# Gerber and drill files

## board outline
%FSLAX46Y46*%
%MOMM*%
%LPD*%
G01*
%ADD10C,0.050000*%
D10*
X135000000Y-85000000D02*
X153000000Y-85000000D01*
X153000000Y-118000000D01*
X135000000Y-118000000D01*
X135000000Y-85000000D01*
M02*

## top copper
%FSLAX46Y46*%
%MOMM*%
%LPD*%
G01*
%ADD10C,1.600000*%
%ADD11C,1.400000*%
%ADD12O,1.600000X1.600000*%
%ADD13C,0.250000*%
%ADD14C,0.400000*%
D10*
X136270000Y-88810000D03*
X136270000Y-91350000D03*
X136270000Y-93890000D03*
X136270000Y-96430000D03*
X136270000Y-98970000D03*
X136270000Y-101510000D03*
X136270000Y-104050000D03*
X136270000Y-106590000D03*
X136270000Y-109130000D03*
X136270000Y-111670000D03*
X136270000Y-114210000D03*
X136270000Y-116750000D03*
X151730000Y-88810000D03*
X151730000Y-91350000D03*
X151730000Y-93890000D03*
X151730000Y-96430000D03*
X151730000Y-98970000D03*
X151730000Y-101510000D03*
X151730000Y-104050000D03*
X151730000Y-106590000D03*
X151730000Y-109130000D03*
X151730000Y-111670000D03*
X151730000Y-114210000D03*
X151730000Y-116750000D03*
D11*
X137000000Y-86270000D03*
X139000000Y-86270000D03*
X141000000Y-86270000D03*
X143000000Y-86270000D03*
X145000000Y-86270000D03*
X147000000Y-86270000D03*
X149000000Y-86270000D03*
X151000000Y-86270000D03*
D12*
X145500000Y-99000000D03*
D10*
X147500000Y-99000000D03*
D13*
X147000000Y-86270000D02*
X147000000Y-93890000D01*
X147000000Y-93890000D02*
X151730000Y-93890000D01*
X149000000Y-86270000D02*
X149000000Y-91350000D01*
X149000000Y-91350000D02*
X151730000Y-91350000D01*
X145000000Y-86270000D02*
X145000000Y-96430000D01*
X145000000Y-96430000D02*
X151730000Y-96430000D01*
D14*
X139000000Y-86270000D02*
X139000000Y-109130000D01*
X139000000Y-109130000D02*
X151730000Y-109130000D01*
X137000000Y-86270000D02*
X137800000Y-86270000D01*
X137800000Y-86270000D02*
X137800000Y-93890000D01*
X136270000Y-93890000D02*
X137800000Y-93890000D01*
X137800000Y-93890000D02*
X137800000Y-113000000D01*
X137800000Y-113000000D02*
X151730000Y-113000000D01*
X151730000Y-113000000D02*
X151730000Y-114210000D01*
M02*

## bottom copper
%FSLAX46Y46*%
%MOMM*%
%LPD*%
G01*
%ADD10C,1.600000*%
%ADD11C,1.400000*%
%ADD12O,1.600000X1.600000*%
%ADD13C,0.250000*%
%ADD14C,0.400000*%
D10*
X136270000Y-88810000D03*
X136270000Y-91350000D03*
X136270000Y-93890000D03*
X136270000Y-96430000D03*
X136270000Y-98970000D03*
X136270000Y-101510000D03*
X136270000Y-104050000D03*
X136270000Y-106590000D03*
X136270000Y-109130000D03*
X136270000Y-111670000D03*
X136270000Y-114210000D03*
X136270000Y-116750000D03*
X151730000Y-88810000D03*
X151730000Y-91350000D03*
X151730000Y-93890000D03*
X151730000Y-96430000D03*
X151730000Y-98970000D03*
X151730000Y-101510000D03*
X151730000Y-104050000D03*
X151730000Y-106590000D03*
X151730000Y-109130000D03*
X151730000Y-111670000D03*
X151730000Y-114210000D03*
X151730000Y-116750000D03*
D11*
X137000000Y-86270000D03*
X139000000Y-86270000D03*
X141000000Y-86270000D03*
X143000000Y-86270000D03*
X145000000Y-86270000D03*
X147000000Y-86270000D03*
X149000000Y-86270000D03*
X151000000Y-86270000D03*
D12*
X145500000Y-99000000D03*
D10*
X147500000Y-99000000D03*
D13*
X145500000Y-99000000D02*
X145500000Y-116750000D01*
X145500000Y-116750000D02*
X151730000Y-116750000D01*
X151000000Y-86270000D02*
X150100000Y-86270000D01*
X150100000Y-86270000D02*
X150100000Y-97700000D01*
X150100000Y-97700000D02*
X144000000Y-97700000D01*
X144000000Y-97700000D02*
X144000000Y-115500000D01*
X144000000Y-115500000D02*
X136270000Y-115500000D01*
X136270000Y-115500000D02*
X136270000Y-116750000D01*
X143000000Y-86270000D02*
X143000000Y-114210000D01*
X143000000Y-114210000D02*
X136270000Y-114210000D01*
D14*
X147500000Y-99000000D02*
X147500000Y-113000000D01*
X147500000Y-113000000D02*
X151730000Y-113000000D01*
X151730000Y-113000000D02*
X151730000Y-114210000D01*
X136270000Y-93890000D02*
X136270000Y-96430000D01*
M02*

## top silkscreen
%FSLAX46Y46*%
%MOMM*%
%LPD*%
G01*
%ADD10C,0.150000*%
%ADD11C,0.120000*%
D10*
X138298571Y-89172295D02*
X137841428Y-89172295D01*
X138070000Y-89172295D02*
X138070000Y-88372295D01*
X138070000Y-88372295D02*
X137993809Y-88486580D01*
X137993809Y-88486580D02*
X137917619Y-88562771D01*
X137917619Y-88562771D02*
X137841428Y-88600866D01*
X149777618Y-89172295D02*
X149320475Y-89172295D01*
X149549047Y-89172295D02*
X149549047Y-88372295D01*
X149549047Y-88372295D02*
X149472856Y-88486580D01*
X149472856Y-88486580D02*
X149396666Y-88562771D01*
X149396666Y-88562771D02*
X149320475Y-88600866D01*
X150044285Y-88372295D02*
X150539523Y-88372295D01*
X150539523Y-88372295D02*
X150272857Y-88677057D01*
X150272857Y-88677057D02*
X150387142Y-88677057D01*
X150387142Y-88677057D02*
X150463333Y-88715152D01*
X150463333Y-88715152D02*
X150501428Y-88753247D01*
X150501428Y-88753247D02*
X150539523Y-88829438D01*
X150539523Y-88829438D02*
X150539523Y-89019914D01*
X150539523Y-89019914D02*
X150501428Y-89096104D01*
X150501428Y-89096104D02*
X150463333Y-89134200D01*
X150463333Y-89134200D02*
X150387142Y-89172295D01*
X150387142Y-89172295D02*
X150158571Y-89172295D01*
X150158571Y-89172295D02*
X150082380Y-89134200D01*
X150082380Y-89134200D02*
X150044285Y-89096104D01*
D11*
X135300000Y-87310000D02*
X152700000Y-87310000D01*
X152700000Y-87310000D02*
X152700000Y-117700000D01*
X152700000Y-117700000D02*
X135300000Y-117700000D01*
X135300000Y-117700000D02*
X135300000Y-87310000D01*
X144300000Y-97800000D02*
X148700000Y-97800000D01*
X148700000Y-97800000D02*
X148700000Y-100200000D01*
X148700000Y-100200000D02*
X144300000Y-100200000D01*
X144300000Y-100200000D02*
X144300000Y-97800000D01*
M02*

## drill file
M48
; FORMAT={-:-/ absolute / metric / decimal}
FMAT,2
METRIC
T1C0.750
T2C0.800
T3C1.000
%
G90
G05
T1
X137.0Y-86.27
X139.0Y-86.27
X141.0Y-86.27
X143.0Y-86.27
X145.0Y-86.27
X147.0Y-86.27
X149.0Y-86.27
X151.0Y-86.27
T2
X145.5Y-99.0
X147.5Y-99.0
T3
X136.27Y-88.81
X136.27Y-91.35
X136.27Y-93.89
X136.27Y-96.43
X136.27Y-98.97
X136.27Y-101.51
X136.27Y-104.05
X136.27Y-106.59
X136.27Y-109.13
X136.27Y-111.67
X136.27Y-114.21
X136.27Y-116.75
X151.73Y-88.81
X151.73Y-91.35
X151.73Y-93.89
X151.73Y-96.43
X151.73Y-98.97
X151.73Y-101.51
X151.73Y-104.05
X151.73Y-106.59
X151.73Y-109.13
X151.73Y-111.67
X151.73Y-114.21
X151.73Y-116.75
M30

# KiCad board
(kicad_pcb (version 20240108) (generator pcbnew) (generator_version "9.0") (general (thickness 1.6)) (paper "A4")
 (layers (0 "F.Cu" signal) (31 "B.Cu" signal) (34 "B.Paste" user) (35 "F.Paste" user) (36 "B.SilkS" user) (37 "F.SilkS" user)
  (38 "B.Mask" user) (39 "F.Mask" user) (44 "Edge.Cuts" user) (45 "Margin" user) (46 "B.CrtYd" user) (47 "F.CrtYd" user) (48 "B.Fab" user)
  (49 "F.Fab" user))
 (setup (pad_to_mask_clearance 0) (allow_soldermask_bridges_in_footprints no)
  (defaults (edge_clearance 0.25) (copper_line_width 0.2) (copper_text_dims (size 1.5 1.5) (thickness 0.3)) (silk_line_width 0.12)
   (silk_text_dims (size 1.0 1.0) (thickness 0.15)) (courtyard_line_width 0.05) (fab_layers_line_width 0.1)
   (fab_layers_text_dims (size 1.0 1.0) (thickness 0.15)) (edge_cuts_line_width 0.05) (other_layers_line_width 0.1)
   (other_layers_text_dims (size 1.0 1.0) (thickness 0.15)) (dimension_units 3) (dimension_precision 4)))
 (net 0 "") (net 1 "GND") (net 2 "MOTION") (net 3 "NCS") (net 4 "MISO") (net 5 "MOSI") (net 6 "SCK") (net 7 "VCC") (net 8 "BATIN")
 (gr_rect (start 135.0000 85.0000) (end 153.0000 118.0000) (stroke (width 0.05) (type default)) (layer "Edge.Cuts"))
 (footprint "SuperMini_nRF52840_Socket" (layer "F.Cu") (at 135.0000 85.0000)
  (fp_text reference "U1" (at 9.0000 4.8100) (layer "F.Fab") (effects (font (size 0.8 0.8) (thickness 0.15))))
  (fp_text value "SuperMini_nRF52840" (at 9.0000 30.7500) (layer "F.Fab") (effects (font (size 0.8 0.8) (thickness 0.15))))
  (pad "1" thru_hole circle (at 1.2700 3.8100) (size 1.6000 1.6000) (drill 1.0000) (layers "*.Cu" "*.Mask"))
  (pad "2" thru_hole circle (at 1.2700 6.3500) (size 1.6000 1.6000) (drill 1.0000) (layers "*.Cu" "*.Mask"))
  (pad "3" thru_hole circle (at 1.2700 8.8900) (size 1.6000 1.6000) (drill 1.0000) (layers "*.Cu" "*.Mask") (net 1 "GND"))
  (pad "4" thru_hole circle (at 1.2700 11.4300) (size 1.6000 1.6000) (drill 1.0000) (layers "*.Cu" "*.Mask") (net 1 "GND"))
  (pad "5" thru_hole circle (at 1.2700 13.9700) (size 1.6000 1.6000) (drill 1.0000) (layers "*.Cu" "*.Mask"))
  (pad "6" thru_hole circle (at 1.2700 16.5100) (size 1.6000 1.6000) (drill 1.0000) (layers "*.Cu" "*.Mask"))
  (pad "7" thru_hole circle (at 1.2700 19.0500) (size 1.6000 1.6000) (drill 1.0000) (layers "*.Cu" "*.Mask"))
  (pad "8" thru_hole circle (at 1.2700 21.5900) (size 1.6000 1.6000) (drill 1.0000) (layers "*.Cu" "*.Mask"))
  (pad "9" thru_hole circle (at 1.2700 24.1300) (size 1.6000 1.6000) (drill 1.0000) (layers "*.Cu" "*.Mask"))
  (pad "10" thru_hole circle (at 1.2700 26.6700) (size 1.6000 1.6000) (drill 1.0000) (layers "*.Cu" "*.Mask"))
  (pad "11" thru_hole circle (at 1.2700 29.2100) (size 1.6000 1.6000) (drill 1.0000) (layers "*.Cu" "*.Mask") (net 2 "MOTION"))
  (pad "12" thru_hole circle (at 1.2700 31.7500) (size 1.6000 1.6000) (drill 1.0000) (layers "*.Cu" "*.Mask") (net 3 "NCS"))
  (pad "13" thru_hole circle (at 16.7300 3.8100) (size 1.6000 1.6000) (drill 1.0000) (layers "*.Cu" "*.Mask"))
  (pad "14" thru_hole circle (at 16.7300 6.3500) (size 1.6000 1.6000) (drill 1.0000) (layers "*.Cu" "*.Mask") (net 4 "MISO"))
  (pad "15" thru_hole circle (at 16.7300 8.8900) (size 1.6000 1.6000) (drill 1.0000) (layers "*.Cu" "*.Mask") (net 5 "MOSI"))
  (pad "16" thru_hole circle (at 16.7300 11.4300) (size 1.6000 1.6000) (drill 1.0000) (layers "*.Cu" "*.Mask") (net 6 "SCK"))
  (pad "17" thru_hole circle (at 16.7300 13.9700) (size 1.6000 1.6000) (drill 1.0000) (layers "*.Cu" "*.Mask"))
  (pad "18" thru_hole circle (at 16.7300 16.5100) (size 1.6000 1.6000) (drill 1.0000) (layers "*.Cu" "*.Mask"))
  (pad "19" thru_hole circle (at 16.7300 19.0500) (size 1.6000 1.6000) (drill 1.0000) (layers "*.Cu" "*.Mask"))
  (pad "20" thru_hole circle (at 16.7300 21.5900) (size 1.6000 1.6000) (drill 1.0000) (layers "*.Cu" "*.Mask"))
  (pad "21" thru_hole circle (at 16.7300 24.1300) (size 1.6000 1.6000) (drill 1.0000) (layers "*.Cu" "*.Mask") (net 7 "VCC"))
  (pad "22" thru_hole circle (at 16.7300 26.6700) (size 1.6000 1.6000) (drill 1.0000) (layers "*.Cu" "*.Mask"))
  (pad "23" thru_hole circle (at 16.7300 29.2100) (size 1.6000 1.6000) (drill 1.0000) (layers "*.Cu" "*.Mask") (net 1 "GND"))
  (pad "24" thru_hole circle (at 16.7300 31.7500) (size 1.6000 1.6000) (drill 1.0000) (layers "*.Cu" "*.Mask") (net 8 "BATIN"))
  (fp_line (start 0.3000 2.3100) (end 17.7000 2.3100) (stroke (width 0.1200) (type default)) (layer "F.SilkS"))
  (fp_line (start 17.7000 2.3100) (end 17.7000 32.7000) (stroke (width 0.1200) (type default)) (layer "F.SilkS"))
  (fp_line (start 17.7000 32.7000) (end 0.3000 32.7000) (stroke (width 0.1200) (type default)) (layer "F.SilkS"))
  (fp_line (start 0.3000 32.7000) (end 0.3000 2.3100) (stroke (width 0.1200) (type default)) (layer "F.SilkS"))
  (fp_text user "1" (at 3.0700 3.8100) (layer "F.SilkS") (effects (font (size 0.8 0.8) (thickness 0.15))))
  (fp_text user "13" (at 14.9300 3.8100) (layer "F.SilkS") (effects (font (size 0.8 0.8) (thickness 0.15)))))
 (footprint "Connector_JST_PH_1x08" (layer "F.Cu") (at 135.0000 85.0000)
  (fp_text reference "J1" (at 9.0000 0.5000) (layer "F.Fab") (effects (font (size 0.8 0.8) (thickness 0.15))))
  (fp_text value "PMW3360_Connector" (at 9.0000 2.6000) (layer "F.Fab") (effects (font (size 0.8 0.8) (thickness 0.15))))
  (pad "1" thru_hole circle (at 2.0000 1.2700) (size 1.4000 1.4000) (drill 0.7500) (layers "*.Cu" "*.Mask") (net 1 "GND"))
  (pad "2" thru_hole circle (at 4.0000 1.2700) (size 1.4000 1.4000) (drill 0.7500) (layers "*.Cu" "*.Mask") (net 7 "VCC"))
  (pad "3" thru_hole circle (at 6.0000 1.2700) (size 1.4000 1.4000) (drill 0.7500) (layers "*.Cu" "*.Mask"))
  (pad "4" thru_hole circle (at 8.0000 1.2700) (size 1.4000 1.4000) (drill 0.7500) (layers "*.Cu" "*.Mask") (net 2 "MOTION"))
  (pad "5" thru_hole circle (at 10.0000 1.2700) (size 1.4000 1.4000) (drill 0.7500) (layers "*.Cu" "*.Mask") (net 6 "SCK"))
  (pad "6" thru_hole circle (at 12.0000 1.2700) (size 1.4000 1.4000) (drill 0.7500) (layers "*.Cu" "*.Mask") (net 5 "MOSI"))
  (pad "7" thru_hole circle (at 14.0000 1.2700) (size 1.4000 1.4000) (drill 0.7500) (layers "*.Cu" "*.Mask") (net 4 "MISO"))
  (pad "8" thru_hole circle (at 16.0000 1.2700) (size 1.4000 1.4000) (drill 0.7500) (layers "*.Cu" "*.Mask") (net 3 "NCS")))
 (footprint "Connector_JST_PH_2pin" (layer "F.Cu") (at 135.0000 85.0000)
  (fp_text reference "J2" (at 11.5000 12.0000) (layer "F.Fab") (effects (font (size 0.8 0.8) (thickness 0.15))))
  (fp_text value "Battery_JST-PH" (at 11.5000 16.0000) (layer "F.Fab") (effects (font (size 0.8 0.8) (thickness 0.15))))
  (pad "1" thru_hole oval (at 10.5000 14.0000) (size 1.6000 1.6000) (drill 0.8000) (layers "*.Cu" "*.Mask") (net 8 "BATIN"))
  (pad "2" thru_hole circle (at 12.5000 14.0000) (size 1.6000 1.6000) (drill 0.8000) (layers "*.Cu" "*.Mask") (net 1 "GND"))
  (fp_line (start 9.3000 12.8000) (end 13.7000 12.8000) (stroke (width 0.1200) (type default)) (layer "F.SilkS"))
  (fp_line (start 13.7000 12.8000) (end 13.7000 15.2000) (stroke (width 0.1200) (type default)) (layer "F.SilkS"))
  (fp_line (start 13.7000 15.2000) (end 9.3000 15.2000) (stroke (width 0.1200) (type default)) (layer "F.SilkS"))
  (fp_line (start 9.3000 15.2000) (end 9.3000 12.8000) (stroke (width 0.1200) (type default)) (layer "F.SilkS")))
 (segment (start 147.0000 86.2700) (end 147.0000 93.8900) (width 0.2500) (layer "F.Cu") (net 5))
 (segment (start 147.0000 93.8900) (end 151.7300 93.8900) (width 0.2500) (layer "F.Cu") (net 5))
 (segment (start 149.0000 86.2700) (end 149.0000 91.3500) (width 0.2500) (layer "F.Cu") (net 4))
 (segment (start 149.0000 91.3500) (end 151.7300 91.3500) (width 0.2500) (layer "F.Cu") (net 4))
 (segment (start 145.0000 86.2700) (end 145.0000 96.4300) (width 0.2500) (layer "F.Cu") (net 6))
 (segment (start 145.0000 96.4300) (end 151.7300 96.4300) (width 0.2500) (layer "F.Cu") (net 6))
 (segment (start 139.0000 86.2700) (end 139.0000 109.1300) (width 0.4000) (layer "F.Cu") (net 7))
 (segment (start 139.0000 109.1300) (end 151.7300 109.1300) (width 0.4000) (layer "F.Cu") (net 7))
 (segment (start 145.5000 99.0000) (end 145.5000 116.7500) (width 0.2500) (layer "B.Cu") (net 8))
 (segment (start 145.5000 116.7500) (end 151.7300 116.7500) (width 0.2500) (layer "B.Cu") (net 8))
 (segment (start 151.0000 86.2700) (end 150.1000 86.2700) (width 0.2500) (layer "B.Cu") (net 3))
 (segment (start 150.1000 86.2700) (end 150.1000 97.7000) (width 0.2500) (layer "B.Cu") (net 3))
 (segment (start 150.1000 97.7000) (end 144.0000 97.7000) (width 0.2500) (layer "B.Cu") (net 3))
 (segment (start 144.0000 97.7000) (end 144.0000 115.5000) (width 0.2500) (layer "B.Cu") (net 3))
 (segment (start 144.0000 115.5000) (end 136.2700 115.5000) (width 0.2500) (layer "B.Cu") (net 3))
 (segment (start 136.2700 115.5000) (end 136.2700 116.7500) (width 0.2500) (layer "B.Cu") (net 3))
 (segment (start 143.0000 86.2700) (end 143.0000 114.2100) (width 0.2500) (layer "B.Cu") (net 2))
 (segment (start 143.0000 114.2100) (end 136.2700 114.2100) (width 0.2500) (layer "B.Cu") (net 2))
 (segment (start 137.0000 86.2700) (end 137.8000 86.2700) (width 0.4000) (layer "F.Cu") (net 1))
 (segment (start 137.8000 86.2700) (end 137.8000 93.8900) (width 0.4000) (layer "F.Cu") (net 1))
 (segment (start 136.2700 93.8900) (end 137.8000 93.8900) (width 0.4000) (layer "F.Cu") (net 1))
 (segment (start 137.8000 93.8900) (end 137.8000 113.0000) (width 0.4000) (layer "F.Cu") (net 1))
 (segment (start 137.8000 113.0000) (end 151.7300 113.0000) (width 0.4000) (layer "F.Cu") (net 1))
 (segment (start 151.7300 113.0000) (end 151.7300 114.2100) (width 0.4000) (layer "F.Cu") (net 1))
 (segment (start 147.5000 99.0000) (end 147.5000 113.0000) (width 0.4000) (layer "B.Cu") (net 1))
 (segment (start 147.5000 113.0000) (end 151.7300 113.0000) (width 0.4000) (layer "B.Cu") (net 1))
 (segment (start 151.7300 113.0000) (end 151.7300 114.2100) (width 0.4000) (layer "B.Cu") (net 1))
 (segment (start 136.2700 93.8900) (end 136.2700 96.4300) (width 0.4000) (layer "B.Cu") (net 1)))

